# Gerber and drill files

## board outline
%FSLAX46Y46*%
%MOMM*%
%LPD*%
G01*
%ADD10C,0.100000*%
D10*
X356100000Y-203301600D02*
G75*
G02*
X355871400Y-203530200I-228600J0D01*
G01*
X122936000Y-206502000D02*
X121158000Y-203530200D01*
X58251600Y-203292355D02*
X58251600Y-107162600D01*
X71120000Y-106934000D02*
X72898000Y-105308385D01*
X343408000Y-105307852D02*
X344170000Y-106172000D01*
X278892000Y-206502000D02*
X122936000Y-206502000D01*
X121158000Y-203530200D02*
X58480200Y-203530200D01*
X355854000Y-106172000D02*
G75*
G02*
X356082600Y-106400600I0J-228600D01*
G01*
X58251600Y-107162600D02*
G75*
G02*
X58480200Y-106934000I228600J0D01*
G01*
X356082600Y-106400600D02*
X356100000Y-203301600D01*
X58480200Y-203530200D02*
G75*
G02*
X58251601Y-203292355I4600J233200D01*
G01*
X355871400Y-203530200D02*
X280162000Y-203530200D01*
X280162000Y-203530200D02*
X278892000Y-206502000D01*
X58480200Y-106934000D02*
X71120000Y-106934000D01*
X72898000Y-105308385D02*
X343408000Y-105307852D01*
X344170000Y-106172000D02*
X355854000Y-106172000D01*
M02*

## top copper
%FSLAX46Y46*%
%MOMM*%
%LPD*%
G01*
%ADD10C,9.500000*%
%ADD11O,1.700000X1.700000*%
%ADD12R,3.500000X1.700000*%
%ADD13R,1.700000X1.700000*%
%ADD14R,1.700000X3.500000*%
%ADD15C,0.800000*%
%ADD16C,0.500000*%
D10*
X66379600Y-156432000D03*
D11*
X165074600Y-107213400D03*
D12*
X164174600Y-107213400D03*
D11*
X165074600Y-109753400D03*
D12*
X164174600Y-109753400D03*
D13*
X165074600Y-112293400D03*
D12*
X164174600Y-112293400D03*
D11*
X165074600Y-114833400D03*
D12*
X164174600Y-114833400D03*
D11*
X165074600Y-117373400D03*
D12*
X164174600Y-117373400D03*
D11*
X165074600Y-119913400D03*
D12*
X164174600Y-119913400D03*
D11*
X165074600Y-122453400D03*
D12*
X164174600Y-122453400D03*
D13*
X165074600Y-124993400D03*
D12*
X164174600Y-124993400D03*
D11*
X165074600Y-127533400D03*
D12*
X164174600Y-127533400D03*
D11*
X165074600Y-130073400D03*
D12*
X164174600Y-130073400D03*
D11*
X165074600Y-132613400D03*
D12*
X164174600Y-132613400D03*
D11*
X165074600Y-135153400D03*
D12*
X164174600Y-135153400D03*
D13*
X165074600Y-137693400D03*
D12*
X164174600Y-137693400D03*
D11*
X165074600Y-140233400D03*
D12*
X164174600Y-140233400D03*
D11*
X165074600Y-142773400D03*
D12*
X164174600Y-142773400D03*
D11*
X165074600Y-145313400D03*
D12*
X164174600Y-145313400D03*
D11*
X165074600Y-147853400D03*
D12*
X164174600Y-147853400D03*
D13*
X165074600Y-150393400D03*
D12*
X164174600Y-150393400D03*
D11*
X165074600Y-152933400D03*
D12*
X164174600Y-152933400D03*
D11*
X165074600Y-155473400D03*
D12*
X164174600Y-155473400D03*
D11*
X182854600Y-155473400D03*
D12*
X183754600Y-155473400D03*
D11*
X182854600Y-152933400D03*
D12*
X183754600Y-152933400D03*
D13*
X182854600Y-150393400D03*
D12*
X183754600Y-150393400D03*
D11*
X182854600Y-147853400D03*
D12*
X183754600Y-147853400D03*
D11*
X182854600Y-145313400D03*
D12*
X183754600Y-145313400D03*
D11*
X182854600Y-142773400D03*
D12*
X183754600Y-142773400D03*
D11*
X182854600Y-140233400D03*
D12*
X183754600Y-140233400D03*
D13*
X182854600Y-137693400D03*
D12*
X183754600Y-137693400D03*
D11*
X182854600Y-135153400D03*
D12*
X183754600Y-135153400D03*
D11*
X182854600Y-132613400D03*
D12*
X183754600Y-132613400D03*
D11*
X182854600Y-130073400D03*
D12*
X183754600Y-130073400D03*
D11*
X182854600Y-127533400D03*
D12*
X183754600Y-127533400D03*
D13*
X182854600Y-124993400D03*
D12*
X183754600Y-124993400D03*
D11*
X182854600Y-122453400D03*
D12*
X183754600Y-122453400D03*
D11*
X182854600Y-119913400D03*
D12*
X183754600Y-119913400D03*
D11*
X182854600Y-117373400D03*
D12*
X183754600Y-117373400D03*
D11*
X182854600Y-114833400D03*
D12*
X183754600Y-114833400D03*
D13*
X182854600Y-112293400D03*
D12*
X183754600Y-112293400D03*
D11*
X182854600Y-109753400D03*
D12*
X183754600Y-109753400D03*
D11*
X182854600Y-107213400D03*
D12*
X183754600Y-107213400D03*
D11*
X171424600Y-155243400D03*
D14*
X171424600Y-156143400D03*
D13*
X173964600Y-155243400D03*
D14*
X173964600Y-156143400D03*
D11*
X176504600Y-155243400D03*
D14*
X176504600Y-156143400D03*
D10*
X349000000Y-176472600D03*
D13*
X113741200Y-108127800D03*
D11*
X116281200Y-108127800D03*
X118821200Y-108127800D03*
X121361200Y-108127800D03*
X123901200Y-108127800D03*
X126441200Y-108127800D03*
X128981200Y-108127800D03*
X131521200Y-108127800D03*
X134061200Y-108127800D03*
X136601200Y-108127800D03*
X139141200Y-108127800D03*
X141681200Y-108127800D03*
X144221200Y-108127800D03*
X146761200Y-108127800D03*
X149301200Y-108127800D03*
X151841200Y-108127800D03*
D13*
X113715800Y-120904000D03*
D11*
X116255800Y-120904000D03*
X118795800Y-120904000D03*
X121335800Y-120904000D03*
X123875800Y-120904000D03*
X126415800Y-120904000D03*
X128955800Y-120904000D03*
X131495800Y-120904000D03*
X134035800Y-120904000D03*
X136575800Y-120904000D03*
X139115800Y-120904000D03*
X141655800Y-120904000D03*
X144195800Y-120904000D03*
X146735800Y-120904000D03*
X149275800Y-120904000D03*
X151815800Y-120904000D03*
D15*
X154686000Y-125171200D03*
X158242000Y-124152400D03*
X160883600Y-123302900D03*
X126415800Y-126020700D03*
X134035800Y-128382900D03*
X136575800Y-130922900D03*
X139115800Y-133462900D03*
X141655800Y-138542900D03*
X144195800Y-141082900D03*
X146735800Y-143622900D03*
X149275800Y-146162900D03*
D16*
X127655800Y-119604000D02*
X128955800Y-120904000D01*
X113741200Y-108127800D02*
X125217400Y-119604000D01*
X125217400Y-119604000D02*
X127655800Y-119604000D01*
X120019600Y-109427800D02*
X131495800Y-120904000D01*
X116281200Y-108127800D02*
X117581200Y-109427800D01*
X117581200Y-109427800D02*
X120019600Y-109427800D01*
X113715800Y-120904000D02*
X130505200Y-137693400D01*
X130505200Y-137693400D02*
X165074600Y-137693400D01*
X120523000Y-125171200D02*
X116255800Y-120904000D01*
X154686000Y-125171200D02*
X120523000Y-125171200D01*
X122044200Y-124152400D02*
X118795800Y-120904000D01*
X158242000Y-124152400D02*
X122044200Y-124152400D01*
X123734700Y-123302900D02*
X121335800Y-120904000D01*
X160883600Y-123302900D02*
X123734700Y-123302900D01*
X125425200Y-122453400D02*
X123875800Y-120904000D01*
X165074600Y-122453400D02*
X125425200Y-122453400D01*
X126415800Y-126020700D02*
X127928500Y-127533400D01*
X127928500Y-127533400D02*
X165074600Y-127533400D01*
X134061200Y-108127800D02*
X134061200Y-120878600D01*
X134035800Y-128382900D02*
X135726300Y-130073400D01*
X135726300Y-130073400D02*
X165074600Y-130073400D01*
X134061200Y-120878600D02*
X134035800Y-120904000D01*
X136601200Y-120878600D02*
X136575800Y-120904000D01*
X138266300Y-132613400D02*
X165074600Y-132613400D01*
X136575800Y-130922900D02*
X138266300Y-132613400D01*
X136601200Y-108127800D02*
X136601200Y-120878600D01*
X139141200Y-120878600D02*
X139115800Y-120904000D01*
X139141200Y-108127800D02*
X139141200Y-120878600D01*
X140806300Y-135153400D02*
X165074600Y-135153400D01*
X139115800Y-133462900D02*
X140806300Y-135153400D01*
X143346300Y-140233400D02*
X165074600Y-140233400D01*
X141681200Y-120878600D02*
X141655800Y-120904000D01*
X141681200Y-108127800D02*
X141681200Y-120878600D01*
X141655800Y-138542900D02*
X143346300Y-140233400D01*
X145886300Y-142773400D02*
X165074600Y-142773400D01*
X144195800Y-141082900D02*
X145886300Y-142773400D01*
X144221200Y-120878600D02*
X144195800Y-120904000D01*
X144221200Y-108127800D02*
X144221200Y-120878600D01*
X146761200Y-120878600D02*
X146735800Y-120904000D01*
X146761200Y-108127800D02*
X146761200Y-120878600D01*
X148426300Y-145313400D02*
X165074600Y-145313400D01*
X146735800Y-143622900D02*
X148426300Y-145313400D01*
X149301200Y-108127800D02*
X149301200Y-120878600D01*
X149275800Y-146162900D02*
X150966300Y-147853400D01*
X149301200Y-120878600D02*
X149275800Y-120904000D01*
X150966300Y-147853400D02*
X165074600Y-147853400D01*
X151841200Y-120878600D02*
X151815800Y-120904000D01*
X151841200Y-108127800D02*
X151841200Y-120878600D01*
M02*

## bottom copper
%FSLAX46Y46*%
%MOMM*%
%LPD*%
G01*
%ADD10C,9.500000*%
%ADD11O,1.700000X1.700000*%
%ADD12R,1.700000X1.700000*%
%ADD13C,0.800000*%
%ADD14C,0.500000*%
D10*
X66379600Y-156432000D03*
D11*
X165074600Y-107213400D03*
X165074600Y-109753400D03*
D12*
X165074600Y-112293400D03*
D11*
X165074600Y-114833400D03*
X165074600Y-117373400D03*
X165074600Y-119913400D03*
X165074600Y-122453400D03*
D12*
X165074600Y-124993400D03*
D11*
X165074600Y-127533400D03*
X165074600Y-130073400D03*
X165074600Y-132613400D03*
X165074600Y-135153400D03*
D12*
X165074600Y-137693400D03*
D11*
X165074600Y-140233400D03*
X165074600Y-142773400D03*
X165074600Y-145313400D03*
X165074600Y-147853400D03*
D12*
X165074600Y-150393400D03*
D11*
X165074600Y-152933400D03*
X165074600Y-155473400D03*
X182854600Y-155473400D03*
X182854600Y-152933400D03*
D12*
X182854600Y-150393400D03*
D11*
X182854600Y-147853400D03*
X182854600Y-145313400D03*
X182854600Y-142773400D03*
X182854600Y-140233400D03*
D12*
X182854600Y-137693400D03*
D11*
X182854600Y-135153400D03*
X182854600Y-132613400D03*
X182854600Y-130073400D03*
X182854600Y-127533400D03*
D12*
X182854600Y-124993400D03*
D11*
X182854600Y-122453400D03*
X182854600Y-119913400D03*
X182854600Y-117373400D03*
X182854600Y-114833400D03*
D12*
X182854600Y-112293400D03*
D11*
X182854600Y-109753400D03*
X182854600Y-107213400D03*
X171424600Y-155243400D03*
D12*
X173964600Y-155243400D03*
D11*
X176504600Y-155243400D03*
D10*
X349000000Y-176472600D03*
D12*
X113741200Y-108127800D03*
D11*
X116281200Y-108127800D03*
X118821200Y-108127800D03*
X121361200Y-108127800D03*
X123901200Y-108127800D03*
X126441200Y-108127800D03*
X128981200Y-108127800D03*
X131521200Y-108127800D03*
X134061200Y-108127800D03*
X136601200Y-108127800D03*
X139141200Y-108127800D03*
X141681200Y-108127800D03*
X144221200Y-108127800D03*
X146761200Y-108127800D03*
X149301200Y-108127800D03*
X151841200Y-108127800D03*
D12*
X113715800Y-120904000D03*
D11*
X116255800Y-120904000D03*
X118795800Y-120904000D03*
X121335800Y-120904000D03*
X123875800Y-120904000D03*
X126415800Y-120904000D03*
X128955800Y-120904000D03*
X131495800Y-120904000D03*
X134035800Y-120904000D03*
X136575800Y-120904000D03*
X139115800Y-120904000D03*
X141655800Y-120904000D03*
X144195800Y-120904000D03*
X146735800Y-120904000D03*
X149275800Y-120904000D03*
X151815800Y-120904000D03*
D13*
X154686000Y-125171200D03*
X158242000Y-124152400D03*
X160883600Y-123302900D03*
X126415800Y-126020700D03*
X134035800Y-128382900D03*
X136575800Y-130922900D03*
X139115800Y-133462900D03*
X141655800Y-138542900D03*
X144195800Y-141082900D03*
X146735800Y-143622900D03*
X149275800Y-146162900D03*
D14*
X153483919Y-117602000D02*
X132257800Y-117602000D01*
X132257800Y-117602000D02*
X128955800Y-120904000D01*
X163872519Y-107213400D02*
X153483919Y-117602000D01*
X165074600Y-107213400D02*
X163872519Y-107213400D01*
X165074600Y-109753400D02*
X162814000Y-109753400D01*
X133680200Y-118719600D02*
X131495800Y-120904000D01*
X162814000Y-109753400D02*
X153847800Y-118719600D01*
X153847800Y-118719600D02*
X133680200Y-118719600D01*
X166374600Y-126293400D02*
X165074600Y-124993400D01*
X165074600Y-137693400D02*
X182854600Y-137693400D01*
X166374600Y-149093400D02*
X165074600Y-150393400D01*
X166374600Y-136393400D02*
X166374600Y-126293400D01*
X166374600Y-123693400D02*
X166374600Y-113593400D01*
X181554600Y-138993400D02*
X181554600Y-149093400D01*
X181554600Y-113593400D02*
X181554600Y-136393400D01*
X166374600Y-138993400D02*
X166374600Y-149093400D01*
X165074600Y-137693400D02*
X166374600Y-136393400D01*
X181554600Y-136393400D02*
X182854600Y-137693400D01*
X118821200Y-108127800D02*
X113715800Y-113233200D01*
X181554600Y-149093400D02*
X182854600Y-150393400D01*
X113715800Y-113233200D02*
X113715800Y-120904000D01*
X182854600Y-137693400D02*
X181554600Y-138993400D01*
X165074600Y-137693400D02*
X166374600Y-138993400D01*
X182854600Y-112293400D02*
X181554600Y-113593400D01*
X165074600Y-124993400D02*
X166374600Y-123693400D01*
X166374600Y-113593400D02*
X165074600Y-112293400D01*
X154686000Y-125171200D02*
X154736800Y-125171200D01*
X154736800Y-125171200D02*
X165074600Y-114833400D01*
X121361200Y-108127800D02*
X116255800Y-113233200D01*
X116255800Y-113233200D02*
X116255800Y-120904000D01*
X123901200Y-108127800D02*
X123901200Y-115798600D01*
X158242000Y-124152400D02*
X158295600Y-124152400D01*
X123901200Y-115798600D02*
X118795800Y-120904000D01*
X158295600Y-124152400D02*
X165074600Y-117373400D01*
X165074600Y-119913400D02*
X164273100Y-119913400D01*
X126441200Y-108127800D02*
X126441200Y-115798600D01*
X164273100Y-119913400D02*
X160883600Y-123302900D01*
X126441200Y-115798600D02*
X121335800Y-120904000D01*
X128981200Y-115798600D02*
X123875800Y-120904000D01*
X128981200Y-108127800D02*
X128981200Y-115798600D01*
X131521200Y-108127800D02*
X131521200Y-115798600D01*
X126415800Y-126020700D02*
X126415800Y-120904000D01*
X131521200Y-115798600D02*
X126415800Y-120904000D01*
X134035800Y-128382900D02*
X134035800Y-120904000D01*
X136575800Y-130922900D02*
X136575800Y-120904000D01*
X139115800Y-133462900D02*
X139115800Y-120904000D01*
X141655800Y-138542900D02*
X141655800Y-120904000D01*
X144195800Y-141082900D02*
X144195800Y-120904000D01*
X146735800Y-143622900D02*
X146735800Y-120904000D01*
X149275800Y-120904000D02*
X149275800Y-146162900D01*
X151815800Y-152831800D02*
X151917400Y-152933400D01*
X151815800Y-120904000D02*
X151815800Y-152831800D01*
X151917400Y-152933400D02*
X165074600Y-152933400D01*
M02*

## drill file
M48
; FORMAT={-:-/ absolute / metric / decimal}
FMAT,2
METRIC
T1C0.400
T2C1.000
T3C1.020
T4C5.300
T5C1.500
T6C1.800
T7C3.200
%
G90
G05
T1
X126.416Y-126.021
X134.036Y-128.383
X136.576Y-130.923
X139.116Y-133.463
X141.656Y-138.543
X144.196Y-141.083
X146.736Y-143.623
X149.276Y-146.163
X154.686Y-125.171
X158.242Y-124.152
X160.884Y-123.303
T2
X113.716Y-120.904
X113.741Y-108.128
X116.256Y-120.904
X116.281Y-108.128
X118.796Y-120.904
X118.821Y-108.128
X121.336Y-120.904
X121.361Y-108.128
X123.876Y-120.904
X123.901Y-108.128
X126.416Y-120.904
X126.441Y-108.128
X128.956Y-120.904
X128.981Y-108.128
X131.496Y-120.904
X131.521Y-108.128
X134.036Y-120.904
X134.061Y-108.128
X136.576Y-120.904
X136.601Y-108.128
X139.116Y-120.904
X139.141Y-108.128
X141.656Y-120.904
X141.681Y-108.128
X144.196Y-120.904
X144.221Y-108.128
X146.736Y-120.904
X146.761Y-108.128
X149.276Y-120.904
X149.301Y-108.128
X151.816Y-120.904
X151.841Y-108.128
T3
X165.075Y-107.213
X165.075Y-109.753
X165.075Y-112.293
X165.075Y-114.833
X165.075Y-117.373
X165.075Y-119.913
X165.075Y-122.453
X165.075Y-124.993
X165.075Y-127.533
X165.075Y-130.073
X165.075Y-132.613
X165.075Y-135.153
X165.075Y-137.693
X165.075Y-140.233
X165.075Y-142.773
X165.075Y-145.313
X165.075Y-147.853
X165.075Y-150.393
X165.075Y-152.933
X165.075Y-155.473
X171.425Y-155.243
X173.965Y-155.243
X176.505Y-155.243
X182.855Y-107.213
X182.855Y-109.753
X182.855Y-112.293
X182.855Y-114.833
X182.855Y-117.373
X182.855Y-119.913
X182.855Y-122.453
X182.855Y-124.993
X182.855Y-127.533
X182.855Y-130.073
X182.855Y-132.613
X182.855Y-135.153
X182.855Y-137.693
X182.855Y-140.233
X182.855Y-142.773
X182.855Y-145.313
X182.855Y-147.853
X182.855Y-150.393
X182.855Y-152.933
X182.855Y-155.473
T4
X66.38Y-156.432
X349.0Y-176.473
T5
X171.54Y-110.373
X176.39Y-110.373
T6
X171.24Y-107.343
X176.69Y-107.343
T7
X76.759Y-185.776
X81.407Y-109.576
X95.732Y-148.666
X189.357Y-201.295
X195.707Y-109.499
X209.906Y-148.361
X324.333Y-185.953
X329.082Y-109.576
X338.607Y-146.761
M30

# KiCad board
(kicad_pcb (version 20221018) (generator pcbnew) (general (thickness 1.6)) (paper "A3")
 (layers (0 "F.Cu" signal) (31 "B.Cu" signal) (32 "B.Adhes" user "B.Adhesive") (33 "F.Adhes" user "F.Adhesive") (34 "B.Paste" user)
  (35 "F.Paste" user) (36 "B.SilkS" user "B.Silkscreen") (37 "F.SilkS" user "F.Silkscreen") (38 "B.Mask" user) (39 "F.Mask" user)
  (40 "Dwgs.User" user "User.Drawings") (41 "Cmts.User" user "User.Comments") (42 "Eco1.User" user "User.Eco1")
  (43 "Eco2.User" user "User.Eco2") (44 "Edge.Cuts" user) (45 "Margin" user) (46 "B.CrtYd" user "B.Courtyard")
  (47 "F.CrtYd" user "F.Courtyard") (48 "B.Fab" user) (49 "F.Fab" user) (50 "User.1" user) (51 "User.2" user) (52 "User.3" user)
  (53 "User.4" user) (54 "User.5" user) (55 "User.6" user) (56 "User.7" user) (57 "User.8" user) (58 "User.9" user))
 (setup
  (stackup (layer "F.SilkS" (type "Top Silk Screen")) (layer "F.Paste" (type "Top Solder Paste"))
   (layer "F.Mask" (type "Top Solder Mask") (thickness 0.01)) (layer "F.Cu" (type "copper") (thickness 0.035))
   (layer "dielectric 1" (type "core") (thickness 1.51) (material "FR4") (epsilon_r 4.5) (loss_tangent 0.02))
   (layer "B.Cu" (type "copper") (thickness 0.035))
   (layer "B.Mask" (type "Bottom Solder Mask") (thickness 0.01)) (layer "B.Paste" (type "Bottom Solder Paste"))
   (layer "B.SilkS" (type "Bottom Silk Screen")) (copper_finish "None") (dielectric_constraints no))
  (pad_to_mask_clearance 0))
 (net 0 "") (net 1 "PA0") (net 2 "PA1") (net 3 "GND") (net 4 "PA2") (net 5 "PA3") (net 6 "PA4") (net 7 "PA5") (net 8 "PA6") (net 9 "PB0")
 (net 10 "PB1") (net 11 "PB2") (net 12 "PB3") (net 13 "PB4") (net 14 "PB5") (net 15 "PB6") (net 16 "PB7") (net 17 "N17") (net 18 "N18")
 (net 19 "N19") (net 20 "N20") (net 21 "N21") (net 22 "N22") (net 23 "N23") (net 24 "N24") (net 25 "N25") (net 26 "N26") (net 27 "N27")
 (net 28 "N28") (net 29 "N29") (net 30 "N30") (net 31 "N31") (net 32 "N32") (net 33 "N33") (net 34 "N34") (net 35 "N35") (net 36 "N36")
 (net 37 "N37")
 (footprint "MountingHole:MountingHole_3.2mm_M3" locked (layer "F.Cu") (at 189.357 201.295)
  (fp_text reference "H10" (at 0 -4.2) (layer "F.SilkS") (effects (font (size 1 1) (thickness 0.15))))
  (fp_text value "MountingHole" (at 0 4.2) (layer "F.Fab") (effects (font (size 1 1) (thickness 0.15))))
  (pad "" np_thru_hole circle locked (at 0 0) (size 3.2 3.2) (drill 3.2) (layers "*.Cu" "*.Mask")))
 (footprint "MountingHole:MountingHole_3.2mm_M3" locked (layer "F.Cu") (at 209.9056 148.3614)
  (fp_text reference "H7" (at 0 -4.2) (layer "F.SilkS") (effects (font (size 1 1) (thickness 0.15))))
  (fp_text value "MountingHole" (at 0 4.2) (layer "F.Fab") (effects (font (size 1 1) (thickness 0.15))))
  (pad "" np_thru_hole circle locked (at 0 0) (size 3.2 3.2) (drill 3.2) (layers "*.Cu" "*.Mask")))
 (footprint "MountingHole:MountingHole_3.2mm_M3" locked (layer "F.Cu") (at 81.407 109.5756)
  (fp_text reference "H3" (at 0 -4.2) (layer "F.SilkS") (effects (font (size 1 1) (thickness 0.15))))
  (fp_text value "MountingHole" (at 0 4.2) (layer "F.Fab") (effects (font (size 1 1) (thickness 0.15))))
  (pad "" np_thru_hole circle locked (at 0 0) (size 3.2 3.2) (drill 3.2) (layers "*.Cu" "*.Mask")))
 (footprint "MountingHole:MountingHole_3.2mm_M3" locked (layer "F.Cu") (at 329.0824 109.5756)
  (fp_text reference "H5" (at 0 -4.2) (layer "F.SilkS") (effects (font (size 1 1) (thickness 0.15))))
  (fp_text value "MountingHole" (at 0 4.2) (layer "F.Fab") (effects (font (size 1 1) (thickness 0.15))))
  (pad "" np_thru_hole circle locked (at 0 0) (size 3.2 3.2) (drill 3.2) (layers "*.Cu" "*.Mask")))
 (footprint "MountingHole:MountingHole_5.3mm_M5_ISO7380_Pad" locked (layer "F.Cu") (at 66.3796 156.432)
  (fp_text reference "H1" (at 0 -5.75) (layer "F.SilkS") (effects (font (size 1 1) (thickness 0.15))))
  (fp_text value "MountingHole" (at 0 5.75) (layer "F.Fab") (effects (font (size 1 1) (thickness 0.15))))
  (pad "1" thru_hole circle locked (at 0 0) (size 9.5 9.5) (drill 5.3) (layers "*.Cu" "*.Mask")))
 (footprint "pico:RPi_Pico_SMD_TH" (layer "F.Cu") (at 173.9646 131.3434)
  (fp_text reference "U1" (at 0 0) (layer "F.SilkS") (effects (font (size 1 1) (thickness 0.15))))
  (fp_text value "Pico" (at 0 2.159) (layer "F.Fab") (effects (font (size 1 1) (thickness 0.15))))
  (pad "" np_thru_hole oval (at -2.725 -24) (size 1.8 1.8) (drill 1.8) (layers "*.Cu" "*.Mask"))
  (pad "" np_thru_hole oval (at -2.425 -20.97) (size 1.5 1.5) (drill 1.5) (layers "*.Cu" "*.Mask"))
  (pad "" np_thru_hole oval (at 2.425 -20.97) (size 1.5 1.5) (drill 1.5) (layers "*.Cu" "*.Mask"))
  (pad "" np_thru_hole oval (at 2.725 -24) (size 1.8 1.8) (drill 1.8) (layers "*.Cu" "*.Mask"))
  (pad "1" thru_hole oval (at -8.89 -24.13) (size 1.7 1.7) (drill 1.02) (layers "*.Cu" "*.Mask") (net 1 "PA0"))
  (pad "1" smd rect (at -8.89 -24.13) (size 3.5 1.7) (drill (offset -0.9 0)) (layers "F.Cu" "F.Mask") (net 1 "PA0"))
  (pad "2" thru_hole oval (at -8.89 -21.59) (size 1.7 1.7) (drill 1.02) (layers "*.Cu" "*.Mask") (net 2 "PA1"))
  (pad "2" smd rect (at -8.89 -21.59) (size 3.5 1.7) (drill (offset -0.9 0)) (layers "F.Cu" "F.Mask") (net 2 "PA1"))
  (pad "3" thru_hole rect (at -8.89 -19.05) (size 1.7 1.7) (drill 1.02) (layers "*.Cu" "*.Mask") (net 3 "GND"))
  (pad "3" smd rect (at -8.89 -19.05) (size 3.5 1.7) (drill (offset -0.9 0)) (layers "F.Cu" "F.Mask") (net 3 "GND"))
  (pad "4" thru_hole oval (at -8.89 -16.51) (size 1.7 1.7) (drill 1.02) (layers "*.Cu" "*.Mask") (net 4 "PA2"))
  (pad "4" smd rect (at -8.89 -16.51) (size 3.5 1.7) (drill (offset -0.9 0)) (layers "F.Cu" "F.Mask") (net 4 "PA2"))
  (pad "5" thru_hole oval (at -8.89 -13.97) (size 1.7 1.7) (drill 1.02) (layers "*.Cu" "*.Mask") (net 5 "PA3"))
  (pad "5" smd rect (at -8.89 -13.97) (size 3.5 1.7) (drill (offset -0.9 0)) (layers "F.Cu" "F.Mask") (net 5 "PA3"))
  (pad "6" thru_hole oval (at -8.89 -11.43) (size 1.7 1.7) (drill 1.02) (layers "*.Cu" "*.Mask") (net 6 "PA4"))
  (pad "6" smd rect (at -8.89 -11.43) (size 3.5 1.7) (drill (offset -0.9 0)) (layers "F.Cu" "F.Mask") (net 6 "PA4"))
  (pad "7" thru_hole oval (at -8.89 -8.89) (size 1.7 1.7) (drill 1.02) (layers "*.Cu" "*.Mask") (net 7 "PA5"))
  (pad "7" smd rect (at -8.89 -8.89) (size 3.5 1.7) (drill (offset -0.9 0)) (layers "F.Cu" "F.Mask") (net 7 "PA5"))
  (pad "8" thru_hole rect (at -8.89 -6.35) (size 1.7 1.7) (drill 1.02) (layers "*.Cu" "*.Mask") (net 3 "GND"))
  (pad "8" smd rect (at -8.89 -6.35) (size 3.5 1.7) (drill (offset -0.9 0)) (layers "F.Cu" "F.Mask") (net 3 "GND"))
  (pad "9" thru_hole oval (at -8.89 -3.81) (size 1.7 1.7) (drill 1.02) (layers "*.Cu" "*.Mask") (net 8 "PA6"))
  (pad "9" smd rect (at -8.89 -3.81) (size 3.5 1.7) (drill (offset -0.9 0)) (layers "F.Cu" "F.Mask") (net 8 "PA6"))
  (pad "10" thru_hole oval (at -8.89 -1.27) (size 1.7 1.7) (drill 1.02) (layers "*.Cu" "*.Mask") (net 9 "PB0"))
  (pad "10" smd rect (at -8.89 -1.27) (size 3.5 1.7) (drill (offset -0.9 0)) (layers "F.Cu" "F.Mask") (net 9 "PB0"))
  (pad "11" thru_hole oval (at -8.89 1.27) (size 1.7 1.7) (drill 1.02) (layers "*.Cu" "*.Mask") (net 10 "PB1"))
  (pad "11" smd rect (at -8.89 1.27) (size 3.5 1.7) (drill (offset -0.9 0)) (layers "F.Cu" "F.Mask") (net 10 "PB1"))
  (pad "12" thru_hole oval (at -8.89 3.81) (size 1.7 1.7) (drill 1.02) (layers "*.Cu" "*.Mask") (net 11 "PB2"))
  (pad "12" smd rect (at -8.89 3.81) (size 3.5 1.7) (drill (offset -0.9 0)) (layers "F.Cu" "F.Mask") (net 11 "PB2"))
  (pad "13" thru_hole rect (at -8.89 6.35) (size 1.7 1.7) (drill 1.02) (layers "*.Cu" "*.Mask") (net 3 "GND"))
  (pad "13" smd rect (at -8.89 6.35) (size 3.5 1.7) (drill (offset -0.9 0)) (layers "F.Cu" "F.Mask") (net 3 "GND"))
  (pad "14" thru_hole oval (at -8.89 8.89) (size 1.7 1.7) (drill 1.02) (layers "*.Cu" "*.Mask") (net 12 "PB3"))
  (pad "14" smd rect (at -8.89 8.89) (size 3.5 1.7) (drill (offset -0.9 0)) (layers "F.Cu" "F.Mask") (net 12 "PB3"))
  (pad "15" thru_hole oval (at -8.89 11.43) (size 1.7 1.7) (drill 1.02) (layers "*.Cu" "*.Mask") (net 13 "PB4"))
  (pad "15" smd rect (at -8.89 11.43) (size 3.5 1.7) (drill (offset -0.9 0)) (layers "F.Cu" "F.Mask") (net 13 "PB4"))
  (pad "16" thru_hole oval (at -8.89 13.97) (size 1.7 1.7) (drill 1.02) (layers "*.Cu" "*.Mask") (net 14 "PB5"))
  (pad "16" smd rect (at -8.89 13.97) (size 3.5 1.7) (drill (offset -0.9 0)) (layers "F.Cu" "F.Mask") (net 14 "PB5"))
  (pad "17" thru_hole oval (at -8.89 16.51) (size 1.7 1.7) (drill 1.02) (layers "*.Cu" "*.Mask") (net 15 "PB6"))
  (pad "17" smd rect (at -8.89 16.51) (size 3.5 1.7) (drill (offset -0.9 0)) (layers "F.Cu" "F.Mask") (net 15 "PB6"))
  (pad "18" thru_hole rect (at -8.89 19.05) (size 1.7 1.7) (drill 1.02) (layers "*.Cu" "*.Mask") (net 3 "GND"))
  (pad "18" smd rect (at -8.89 19.05) (size 3.5 1.7) (drill (offset -0.9 0)) (layers "F.Cu" "F.Mask") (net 3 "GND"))
  (pad "19" thru_hole oval (at -8.89 21.59) (size 1.7 1.7) (drill 1.02) (layers "*.Cu" "*.Mask") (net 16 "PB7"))
  (pad "19" smd rect (at -8.89 21.59) (size 3.5 1.7) (drill (offset -0.9 0)) (layers "F.Cu" "F.Mask") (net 16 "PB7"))
  (pad "20" thru_hole oval (at -8.89 24.13) (size 1.7 1.7) (drill 1.02) (layers "*.Cu" "*.Mask") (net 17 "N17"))
  (pad "20" smd rect (at -8.89 24.13) (size 3.5 1.7) (drill (offset -0.9 0)) (layers "F.Cu" "F.Mask") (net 17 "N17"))
  (pad "21" thru_hole oval (at 8.89 24.13) (size 1.7 1.7) (drill 1.02) (layers "*.Cu" "*.Mask") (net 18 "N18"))
  (pad "21" smd rect (at 8.89 24.13) (size 3.5 1.7) (drill (offset 0.9 0)) (layers "F.Cu" "F.Mask") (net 18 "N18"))
  (pad "22" thru_hole oval (at 8.89 21.59) (size 1.7 1.7) (drill 1.02) (layers "*.Cu" "*.Mask") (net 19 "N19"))
  (pad "22" smd rect (at 8.89 21.59) (size 3.5 1.7) (drill (offset 0.9 0)) (layers "F.Cu" "F.Mask") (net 19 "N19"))
  (pad "23" thru_hole rect (at 8.89 19.05) (size 1.7 1.7) (drill 1.02) (layers "*.Cu" "*.Mask") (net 3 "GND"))
  (pad "23" smd rect (at 8.89 19.05) (size 3.5 1.7) (drill (offset 0.9 0)) (layers "F.Cu" "F.Mask") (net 3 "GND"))
  (pad "24" thru_hole oval (at 8.89 16.51) (size 1.7 1.7) (drill 1.02) (layers "*.Cu" "*.Mask") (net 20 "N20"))
  (pad "24" smd rect (at 8.89 16.51) (size 3.5 1.7) (drill (offset 0.9 0)) (layers "F.Cu" "F.Mask") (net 20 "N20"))
  (pad "25" thru_hole oval (at 8.89 13.97) (size 1.7 1.7) (drill 1.02) (layers "*.Cu" "*.Mask") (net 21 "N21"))
  (pad "25" smd rect (at 8.89 13.97) (size 3.5 1.7) (drill (offset 0.9 0)) (layers "F.Cu" "F.Mask") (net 21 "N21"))
  (pad "26" thru_hole oval (at 8.89 11.43) (size 1.7 1.7) (drill 1.02) (layers "*.Cu" "*.Mask") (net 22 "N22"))
  (pad "26" smd rect (at 8.89 11.43) (size 3.5 1.7) (drill (offset 0.9 0)) (layers "F.Cu" "F.Mask") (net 22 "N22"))
  (pad "27" thru_hole oval (at 8.89 8.89) (size 1.7 1.7) (drill 1.02) (layers "*.Cu" "*.Mask") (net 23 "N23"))
  (pad "27" smd rect (at 8.89 8.89) (size 3.5 1.7) (drill (offset 0.9 0)) (layers "F.Cu" "F.Mask") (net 23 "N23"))
  (pad "28" thru_hole rect (at 8.89 6.35) (size 1.7 1.7) (drill 1.02) (layers "*.Cu" "*.Mask") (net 3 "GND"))
  (pad "28" smd rect (at 8.89 6.35) (size 3.5 1.7) (drill (offset 0.9 0)) (layers "F.Cu" "F.Mask") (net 3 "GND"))
  (pad "29" thru_hole oval (at 8.89 3.81) (size 1.7 1.7) (drill 1.02) (layers "*.Cu" "*.Mask") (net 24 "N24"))
  (pad "29" smd rect (at 8.89 3.81) (size 3.5 1.7) (drill (offset 0.9 0)) (layers "F.Cu" "F.Mask") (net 24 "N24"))
  (pad "30" thru_hole oval (at 8.89 1.27) (size 1.7 1.7) (drill 1.02) (layers "*.Cu" "*.Mask") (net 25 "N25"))
  (pad "30" smd rect (at 8.89 1.27) (size 3.5 1.7) (drill (offset 0.9 0)) (layers "F.Cu" "F.Mask") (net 25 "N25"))
  (pad "31" thru_hole oval (at 8.89 -1.27) (size 1.7 1.7) (drill 1.02) (layers "*.Cu" "*.Mask") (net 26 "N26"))
  (pad "31" smd rect (at 8.89 -1.27) (size 3.5 1.7) (drill (offset 0.9 0)) (layers "F.Cu" "F.Mask") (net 26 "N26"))
  (pad "32" thru_hole oval (at 8.89 -3.81) (size 1.7 1.7) (drill 1.02) (layers "*.Cu" "*.Mask") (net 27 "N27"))
  (pad "32" smd rect (at 8.89 -3.81) (size 3.5 1.7) (drill (offset 0.9 0)) (layers "F.Cu" "F.Mask") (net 27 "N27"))
  (pad "33" thru_hole rect (at 8.89 -6.35) (size 1.7 1.7) (drill 1.02) (layers "*.Cu" "*.Mask") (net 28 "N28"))
  (pad "33" smd rect (at 8.89 -6.35) (size 3.5 1.7) (drill (offset 0.9 0)) (layers "F.Cu" "F.Mask") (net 28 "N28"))
  (pad "34" thru_hole oval (at 8.89 -8.89) (size 1.7 1.7) (drill 1.02) (layers "*.Cu" "*.Mask") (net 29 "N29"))
  (pad "34" smd rect (at 8.89 -8.89) (size 3.5 1.7) (drill (offset 0.9 0)) (layers "F.Cu" "F.Mask") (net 29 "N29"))
  (pad "35" thru_hole oval (at 8.89 -11.43) (size 1.7 1.7) (drill 1.02) (layers "*.Cu" "*.Mask") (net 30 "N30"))
  (pad "35" smd rect (at 8.89 -11.43) (size 3.5 1.7) (drill (offset 0.9 0)) (layers "F.Cu" "F.Mask") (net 30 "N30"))
  (pad "36" thru_hole oval (at 8.89 -13.97) (size 1.7 1.7) (drill 1.02) (layers "*.Cu" "*.Mask") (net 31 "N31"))
  (pad "36" smd rect (at 8.89 -13.97) (size 3.5 1.7) (drill (offset 0.9 0)) (layers "F.Cu" "F.Mask") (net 31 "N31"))
  (pad "37" thru_hole oval (at 8.89 -16.51) (size 1.7 1.7) (drill 1.02) (layers "*.Cu" "*.Mask") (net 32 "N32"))
  (pad "37" smd rect (at 8.89 -16.51) (size 3.5 1.7) (drill (offset 0.9 0)) (layers "F.Cu" "F.Mask") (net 32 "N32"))
  (pad "38" thru_hole rect (at 8.89 -19.05) (size 1.7 1.7) (drill 1.02) (layers "*.Cu" "*.Mask") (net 3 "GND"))
  (pad "38" smd rect (at 8.89 -19.05) (size 3.5 1.7) (drill (offset 0.9 0)) (layers "F.Cu" "F.Mask") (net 3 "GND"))
  (pad "39" thru_hole oval (at 8.89 -21.59) (size 1.7 1.7) (drill 1.02) (layers "*.Cu" "*.Mask") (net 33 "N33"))
  (pad "39" smd rect (at 8.89 -21.59) (size 3.5 1.7) (drill (offset 0.9 0)) (layers "F.Cu" "F.Mask") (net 33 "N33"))
  (pad "40" thru_hole oval (at 8.89 -24.13) (size 1.7 1.7) (drill 1.02) (layers "*.Cu" "*.Mask") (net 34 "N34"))
  (pad "40" smd rect (at 8.89 -24.13) (size 3.5 1.7) (drill (offset 0.9 0)) (layers "F.Cu" "F.Mask") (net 34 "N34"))
  (pad "41" thru_hole oval (at -2.54 23.9) (size 1.7 1.7) (drill 1.02) (layers "*.Cu" "*.Mask") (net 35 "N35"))
  (pad "41" smd rect (at -2.54 23.9 90) (size 3.5 1.7) (drill (offset -0.9 0)) (layers "F.Cu" "F.Mask") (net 35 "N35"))
  (pad "42" thru_hole rect (at 0 23.9) (size 1.7 1.7) (drill 1.02) (layers "*.Cu" "*.Mask") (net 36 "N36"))
  (pad "42" smd rect (at 0 23.9 90) (size 3.5 1.7) (drill (offset -0.9 0)) (layers "F.Cu" "F.Mask") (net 36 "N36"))
  (pad "43" thru_hole oval (at 2.54 23.9) (size 1.7 1.7) (drill 1.02) (layers "*.Cu" "*.Mask") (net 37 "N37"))
  (pad "43" smd rect (at 2.54 23.9 90) (size 3.5 1.7) (drill (offset -0.9 0)) (layers "F.Cu" "F.Mask") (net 37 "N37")))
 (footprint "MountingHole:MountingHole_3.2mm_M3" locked (layer "F.Cu") (at 338.6074 146.7612)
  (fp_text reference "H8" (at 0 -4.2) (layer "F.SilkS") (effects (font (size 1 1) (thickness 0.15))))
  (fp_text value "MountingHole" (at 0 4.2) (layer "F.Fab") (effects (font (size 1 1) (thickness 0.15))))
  (pad "" np_thru_hole circle locked (at 0 0) (size 3.2 3.2) (drill 3.2) (layers "*.Cu" "*.Mask")))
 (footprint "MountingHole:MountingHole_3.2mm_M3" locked (layer "F.Cu") (at 95.732 148.6662)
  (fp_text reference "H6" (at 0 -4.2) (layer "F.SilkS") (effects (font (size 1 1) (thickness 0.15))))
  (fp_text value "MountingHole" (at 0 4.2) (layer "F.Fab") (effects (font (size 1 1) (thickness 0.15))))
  (pad "" np_thru_hole circle locked (at 0 0) (size 3.2 3.2) (drill 3.2) (layers "*.Cu" "*.Mask")))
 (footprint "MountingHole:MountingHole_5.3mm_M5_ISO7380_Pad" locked (layer "F.Cu") (at 349 176.4726)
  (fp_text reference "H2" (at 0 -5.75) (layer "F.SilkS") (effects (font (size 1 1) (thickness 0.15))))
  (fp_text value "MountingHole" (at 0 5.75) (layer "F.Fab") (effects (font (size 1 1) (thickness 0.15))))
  (pad "1" thru_hole circle locked (at 0 0) (size 9.5 9.5) (drill 5.3) (layers "*.Cu" "*.Mask")))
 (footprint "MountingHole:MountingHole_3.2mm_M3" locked (layer "F.Cu") (at 195.707 109.4994)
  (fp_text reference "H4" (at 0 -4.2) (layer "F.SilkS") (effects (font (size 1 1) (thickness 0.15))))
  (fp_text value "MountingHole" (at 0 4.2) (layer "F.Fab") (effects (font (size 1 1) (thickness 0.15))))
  (pad "" np_thru_hole circle locked (at 0 0) (size 3.2 3.2) (drill 3.2) (layers "*.Cu" "*.Mask")))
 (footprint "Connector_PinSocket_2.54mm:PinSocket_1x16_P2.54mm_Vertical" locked (layer "F.Cu") (at 113.7412 108.1278 90)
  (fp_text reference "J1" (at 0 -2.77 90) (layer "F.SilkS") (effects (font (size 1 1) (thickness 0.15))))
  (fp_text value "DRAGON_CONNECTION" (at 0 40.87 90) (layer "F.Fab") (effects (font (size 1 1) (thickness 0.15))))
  (pad "1" thru_hole rect locked (at 0 0 90) (size 1.7 1.7) (drill 1) (layers "*.Cu" "*.Mask") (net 1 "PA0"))
  (pad "2" thru_hole oval locked (at 0 2.54 90) (size 1.7 1.7) (drill 1) (layers "*.Cu" "*.Mask") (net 2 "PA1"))
  (pad "3" thru_hole oval locked (at 0 5.08 90) (size 1.7 1.7) (drill 1) (layers "*.Cu" "*.Mask") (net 3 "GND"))
  (pad "4" thru_hole oval locked (at 0 7.62 90) (size 1.7 1.7) (drill 1) (layers "*.Cu" "*.Mask") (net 4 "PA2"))
  (pad "5" thru_hole oval locked (at 0 10.16 90) (size 1.7 1.7) (drill 1) (layers "*.Cu" "*.Mask") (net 5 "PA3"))
  (pad "6" thru_hole oval locked (at 0 12.7 90) (size 1.7 1.7) (drill 1) (layers "*.Cu" "*.Mask") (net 6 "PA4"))
  (pad "7" thru_hole oval locked (at 0 15.24 90) (size 1.7 1.7) (drill 1) (layers "*.Cu" "*.Mask") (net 7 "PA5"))
  (pad "8" thru_hole oval locked (at 0 17.78 90) (size 1.7 1.7) (drill 1) (layers "*.Cu" "*.Mask") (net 8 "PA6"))
  (pad "9" thru_hole oval locked (at 0 20.32 90) (size 1.7 1.7) (drill 1) (layers "*.Cu" "*.Mask") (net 9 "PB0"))
  (pad "10" thru_hole oval locked (at 0 22.86 90) (size 1.7 1.7) (drill 1) (layers "*.Cu" "*.Mask") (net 10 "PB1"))
  (pad "11" thru_hole oval locked (at 0 25.4 90) (size 1.7 1.7) (drill 1) (layers "*.Cu" "*.Mask") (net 11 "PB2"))
  (pad "12" thru_hole oval locked (at 0 27.94 90) (size 1.7 1.7) (drill 1) (layers "*.Cu" "*.Mask") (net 12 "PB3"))
  (pad "13" thru_hole oval locked (at 0 30.48 90) (size 1.7 1.7) (drill 1) (layers "*.Cu" "*.Mask") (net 13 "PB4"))
  (pad "14" thru_hole oval locked (at 0 33.02 90) (size 1.7 1.7) (drill 1) (layers "*.Cu" "*.Mask") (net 14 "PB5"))
  (pad "15" thru_hole oval locked (at 0 35.56 90) (size 1.7 1.7) (drill 1) (layers "*.Cu" "*.Mask") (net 15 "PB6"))
  (pad "16" thru_hole oval locked (at 0 38.1 90) (size 1.7 1.7) (drill 1) (layers "*.Cu" "*.Mask") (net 16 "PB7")))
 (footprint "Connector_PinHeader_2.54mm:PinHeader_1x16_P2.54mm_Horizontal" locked (layer "F.Cu") (at 113.7158 120.904 90)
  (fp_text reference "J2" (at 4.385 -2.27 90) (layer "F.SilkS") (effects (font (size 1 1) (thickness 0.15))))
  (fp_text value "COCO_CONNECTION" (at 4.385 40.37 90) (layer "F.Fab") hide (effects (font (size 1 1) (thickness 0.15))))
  (pad "1" thru_hole rect locked (at 0 0 90) (size 1.7 1.7) (drill 1) (layers "*.Cu" "*.Mask") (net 3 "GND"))
  (pad "2" thru_hole oval locked (at 0 2.54 90) (size 1.7 1.7) (drill 1) (layers "*.Cu" "*.Mask") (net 4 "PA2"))
  (pad "3" thru_hole oval locked (at 0 5.08 90) (size 1.7 1.7) (drill 1) (layers "*.Cu" "*.Mask") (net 5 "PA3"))
  (pad "4" thru_hole oval locked (at 0 7.62 90) (size 1.7 1.7) (drill 1) (layers "*.Cu" "*.Mask") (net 6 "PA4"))
  (pad "5" thru_hole oval locked (at 0 10.16 90) (size 1.7 1.7) (drill 1) (layers "*.Cu" "*.Mask") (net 7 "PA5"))
  (pad "6" thru_hole oval locked (at 0 12.7 90) (size 1.7 1.7) (drill 1) (layers "*.Cu" "*.Mask") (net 8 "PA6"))
  (pad "7" thru_hole oval locked (at 0 15.24 90) (size 1.7 1.7) (drill 1) (layers "*.Cu" "*.Mask") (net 1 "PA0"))
  (pad "8" thru_hole oval locked (at 0 17.78 90) (size 1.7 1.7) (drill 1) (layers "*.Cu" "*.Mask") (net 2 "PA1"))
  (pad "9" thru_hole oval locked (at 0 20.32 90) (size 1.7 1.7) (drill 1) (layers "*.Cu" "*.Mask") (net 9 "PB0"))
  (pad "10" thru_hole oval locked (at 0 22.86 90) (size 1.7 1.7) (drill 1) (layers "*.Cu" "*.Mask") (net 10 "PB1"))
  (pad "11" thru_hole oval locked (at 0 25.4 90) (size 1.7 1.7) (drill 1) (layers "*.Cu" "*.Mask") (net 11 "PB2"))
  (pad "12" thru_hole oval locked (at 0 27.94 90) (size 1.7 1.7) (drill 1) (layers "*.Cu" "*.Mask") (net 12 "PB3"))
  (pad "13" thru_hole oval locked (at 0 30.48 90) (size 1.7 1.7) (drill 1) (layers "*.Cu" "*.Mask") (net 13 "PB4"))
  (pad "14" thru_hole oval locked (at 0 33.02 90) (size 1.7 1.7) (drill 1) (layers "*.Cu" "*.Mask") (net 14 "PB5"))
  (pad "15" thru_hole oval locked (at 0 35.56 90) (size 1.7 1.7) (drill 1) (layers "*.Cu" "*.Mask") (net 15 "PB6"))
  (pad "16" thru_hole oval locked (at 0 38.1 90) (size 1.7 1.7) (drill 1) (layers "*.Cu" "*.Mask") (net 16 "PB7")))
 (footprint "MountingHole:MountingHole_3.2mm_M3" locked (layer "F.Cu") (at 324.3326 185.9534)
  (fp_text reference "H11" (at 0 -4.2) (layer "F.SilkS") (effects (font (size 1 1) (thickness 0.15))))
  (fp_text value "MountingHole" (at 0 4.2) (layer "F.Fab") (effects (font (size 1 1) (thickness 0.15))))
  (pad "" np_thru_hole circle locked (at 0 0) (size 3.2 3.2) (drill 3.2) (layers "*.Cu" "*.Mask")))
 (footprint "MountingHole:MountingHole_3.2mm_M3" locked (layer "F.Cu") (at 76.7588 185.7756)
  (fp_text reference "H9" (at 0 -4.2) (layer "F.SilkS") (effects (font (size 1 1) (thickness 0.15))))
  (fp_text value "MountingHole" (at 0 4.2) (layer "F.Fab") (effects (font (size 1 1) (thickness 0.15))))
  (pad "" np_thru_hole circle locked (at 0 0) (size 3.2 3.2) (drill 3.2) (layers "*.Cu" "*.Mask")))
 (gr_arc (start 356.1 203.3016) (mid 356.033045 203.463245) (end 355.8714 203.5302) (stroke (width 0.1) (type default)) (layer "Edge.Cuts"))
 (gr_line (start 122.936 206.502) (end 121.158 203.5302) (stroke (width 0.1) (type default)) (layer "Edge.Cuts"))
 (gr_line (start 58.2516 203.292355) (end 58.2516 107.1626) (stroke (width 0.1) (type default)) (layer "Edge.Cuts"))
 (gr_line (start 71.12 106.934) (end 72.898 105.308385) (stroke (width 0.1) (type default)) (layer "Edge.Cuts"))
 (gr_line (start 343.408 105.307852) (end 344.17 106.172) (stroke (width 0.1) (type default)) (layer "Edge.Cuts"))
 (gr_line (start 278.892 206.502) (end 122.936 206.502) (stroke (width 0.1) (type default)) (layer "Edge.Cuts"))
 (gr_line (start 121.158 203.5302) (end 58.4802 203.5302) (stroke (width 0.1) (type default)) (layer "Edge.Cuts"))
 (gr_arc (start 355.854 106.172) (mid 356.015624 106.238962) (end 356.0826 106.4006) (stroke (width 0.1) (type default)) (layer "Edge.Cuts"))
 (gr_arc (start 58.2516 107.1626) (mid 58.318555 107.000955) (end 58.4802 106.934) (stroke (width 0.1) (type default)) (layer "Edge.Cuts"))
 (gr_line (start 356.0826 106.4006) (end 356.1 203.3016) (stroke (width 0.1) (type default)) (layer "Edge.Cuts"))
 (gr_arc (start 58.4802 203.5302) (mid 58.316634 203.458629) (end 58.2516 203.292355) (stroke (width 0.1) (type default))
  (layer "Edge.Cuts"))
 (gr_line (start 355.8714 203.5302) (end 280.162 203.5302) (stroke (width 0.1) (type default)) (layer "Edge.Cuts"))
 (gr_line (start 280.162 203.5302) (end 278.892 206.502) (stroke (width 0.1) (type default)) (layer "Edge.Cuts"))
 (gr_line (start 58.4802 106.934) (end 71.12 106.934) (stroke (width 0.1) (type default)) (layer "Edge.Cuts"))
 (gr_line (start 72.898 105.308385) (end 343.408 105.307852) (stroke (width 0.1) (type default)) (layer "Edge.Cuts"))
 (gr_line (start 344.17 106.172) (end 355.854 106.172) (stroke (width 0.1) (type default)) (layer "Edge.Cuts"))
 (segment (start 127.6558 119.604) (end 128.9558 120.904) (width 0.5) (layer "F.Cu") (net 1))
 (segment (start 113.7412 108.1278) (end 125.2174 119.604) (width 0.5) (layer "F.Cu") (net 1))
 (segment (start 125.2174 119.604) (end 127.6558 119.604) (width 0.5) (layer "F.Cu") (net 1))
 (segment (start 153.483919 117.602) (end 132.2578 117.602) (width 0.5) (layer "B.Cu") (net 1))
 (segment (start 132.2578 117.602) (end 128.9558 120.904) (width 0.5) (layer "B.Cu") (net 1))
 (segment (start 163.872519 107.2134) (end 153.483919 117.602) (width 0.5) (layer "B.Cu") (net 1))
 (segment (start 165.0746 107.2134) (end 163.872519 107.2134) (width 0.5) (layer "B.Cu") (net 1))
 (segment (start 120.0196 109.4278) (end 131.4958 120.904) (width 0.5) (layer "F.Cu") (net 2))
 (segment (start 116.2812 108.1278) (end 117.5812 109.4278) (width 0.5) (layer "F.Cu") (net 2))
 (segment (start 117.5812 109.4278) (end 120.0196 109.4278) (width 0.5) (layer "F.Cu") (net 2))
 (segment (start 165.0746 109.7534) (end 162.814 109.7534) (width 0.5) (layer "B.Cu") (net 2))
 (segment (start 133.6802 118.7196) (end 131.4958 120.904) (width 0.5) (layer "B.Cu") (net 2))
 (segment (start 162.814 109.7534) (end 153.8478 118.7196) (width 0.5) (layer "B.Cu") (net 2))
 (segment (start 153.8478 118.7196) (end 133.6802 118.7196) (width 0.5) (layer "B.Cu") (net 2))
 (segment (start 113.7158 120.904) (end 130.5052 137.6934) (width 0.5) (layer "F.Cu") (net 3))
 (segment (start 130.5052 137.6934) (end 165.0746 137.6934) (width 0.5) (layer "F.Cu") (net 3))
 (segment (start 166.3746 126.2934) (end 165.0746 124.9934) (width 0.5) (layer "B.Cu") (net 3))
 (segment (start 165.0746 137.6934) (end 182.8546 137.6934) (width 0.5) (layer "B.Cu") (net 3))
 (segment (start 166.3746 149.0934) (end 165.0746 150.3934) (width 0.5) (layer "B.Cu") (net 3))
 (segment (start 166.3746 136.3934) (end 166.3746 126.2934) (width 0.5) (layer "B.Cu") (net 3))
 (segment (start 166.3746 123.6934) (end 166.3746 113.5934) (width 0.5) (layer "B.Cu") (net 3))
 (segment (start 181.5546 138.9934) (end 181.5546 149.0934) (width 0.5) (layer "B.Cu") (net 3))
 (segment (start 181.5546 113.5934) (end 181.5546 136.3934) (width 0.5) (layer "B.Cu") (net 3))
 (segment (start 166.3746 138.9934) (end 166.3746 149.0934) (width 0.5) (layer "B.Cu") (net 3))
 (segment (start 165.0746 137.6934) (end 166.3746 136.3934) (width 0.5) (layer "B.Cu") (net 3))
 (segment (start 181.5546 136.3934) (end 182.8546 137.6934) (width 0.5) (layer "B.Cu") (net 3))
 (segment (start 118.8212 108.1278) (end 113.7158 113.2332) (width 0.5) (layer "B.Cu") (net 3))
 (segment (start 181.5546 149.0934) (end 182.8546 150.3934) (width 0.5) (layer "B.Cu") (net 3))
 (segment (start 113.7158 113.2332) (end 113.7158 120.904) (width 0.5) (layer "B.Cu") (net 3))
 (segment (start 182.8546 137.6934) (end 181.5546 138.9934) (width 0.5) (layer "B.Cu") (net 3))
 (segment (start 165.0746 137.6934) (end 166.3746 138.9934) (width 0.5) (layer "B.Cu") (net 3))
 (segment (start 182.8546 112.2934) (end 181.5546 113.5934) (width 0.5) (layer "B.Cu") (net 3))
 (segment (start 165.0746 124.9934) (end 166.3746 123.6934) (width 0.5) (layer "B.Cu") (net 3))
 (segment (start 166.3746 113.5934) (end 165.0746 112.2934) (width 0.5) (layer "B.Cu") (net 3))
 (segment (start 120.523 125.1712) (end 116.2558 120.904) (width 0.5) (layer "F.Cu") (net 4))
 (segment (start 154.686 125.1712) (end 120.523 125.1712) (width 0.5) (layer "F.Cu") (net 4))
 (via (at 154.686 125.1712) (size 0.8) (drill 0.4) (layers "F.Cu" "B.Cu") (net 4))
 (segment (start 154.686 125.1712) (end 154.7368 125.1712) (width 0.5) (layer "B.Cu") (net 4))
 (segment (start 154.7368 125.1712) (end 165.0746 114.8334) (width 0.5) (layer "B.Cu") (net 4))
 (segment (start 121.3612 108.1278) (end 116.2558 113.2332) (width 0.5) (layer "B.Cu") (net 4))
 (segment (start 116.2558 113.2332) (end 116.2558 120.904) (width 0.5) (layer "B.Cu") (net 4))
 (segment (start 122.0442 124.1524) (end 118.7958 120.904) (width 0.5) (layer "F.Cu") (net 5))
 (segment (start 158.242 124.1524) (end 122.0442 124.1524) (width 0.5) (layer "F.Cu") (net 5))
 (via (at 158.242 124.1524) (size 0.8) (drill 0.4) (layers "F.Cu" "B.Cu") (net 5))
 (segment (start 123.9012 108.1278) (end 123.9012 115.7986) (width 0.5) (layer "B.Cu") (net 5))
 (segment (start 158.242 124.1524) (end 158.2956 124.1524) (width 0.5) (layer "B.Cu") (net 5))
 (segment (start 123.9012 115.7986) (end 118.7958 120.904) (width 0.5) (layer "B.Cu") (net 5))
 (segment (start 158.2956 124.1524) (end 165.0746 117.3734) (width 0.5) (layer "B.Cu") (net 5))
 (segment (start 123.7347 123.3029) (end 121.3358 120.904) (width 0.5) (layer "F.Cu") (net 6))
 (segment (start 160.8836 123.3029) (end 123.7347 123.3029) (width 0.5) (layer "F.Cu") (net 6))
 (via (at 160.8836 123.3029) (size 0.8) (drill 0.4) (layers "F.Cu" "B.Cu") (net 6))
 (segment (start 165.0746 119.9134) (end 164.2731 119.9134) (width 0.5) (layer "B.Cu") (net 6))
 (segment (start 126.4412 108.1278) (end 126.4412 115.7986) (width 0.5) (layer "B.Cu") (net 6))
 (segment (start 164.2731 119.9134) (end 160.8836 123.3029) (width 0.5) (layer "B.Cu") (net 6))
 (segment (start 126.4412 115.7986) (end 121.3358 120.904) (width 0.5) (layer "B.Cu") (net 6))
 (segment (start 125.4252 122.4534) (end 123.8758 120.904) (width 0.5) (layer "F.Cu") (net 7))
 (segment (start 165.0746 122.4534) (end 125.4252 122.4534) (width 0.5) (layer "F.Cu") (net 7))
 (segment (start 128.9812 115.7986) (end 123.8758 120.904) (width 0.5) (layer "B.Cu") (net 7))
 (segment (start 128.9812 108.1278) (end 128.9812 115.7986) (width 0.5) (layer "B.Cu") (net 7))
 (segment (start 126.4158 126.0207) (end 127.9285 127.5334) (width 0.5) (layer "F.Cu") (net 8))
 (segment (start 127.9285 127.5334) (end 165.0746 127.5334) (width 0.5) (layer "F.Cu") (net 8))
 (via (at 126.4158 126.0207) (size 0.8) (drill 0.4) (layers "F.Cu" "B.Cu") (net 8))
 (segment (start 131.5212 108.1278) (end 131.5212 115.7986) (width 0.5) (layer "B.Cu") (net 8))
 (segment (start 126.4158 126.0207) (end 126.4158 120.904) (width 0.5) (layer "B.Cu") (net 8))
 (segment (start 131.5212 115.7986) (end 126.4158 120.904) (width 0.5) (layer "B.Cu") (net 8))
 (segment (start 134.0612 108.1278) (end 134.0612 120.8786) (width 0.5) (layer "F.Cu") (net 9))
 (segment (start 134.0358 128.3829) (end 135.7263 130.0734) (width 0.5) (layer "F.Cu") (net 9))
 (segment (start 135.7263 130.0734) (end 165.0746 130.0734) (width 0.5) (layer "F.Cu") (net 9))
 (segment (start 134.0612 120.8786) (end 134.0358 120.904) (width 0.5) (layer "F.Cu") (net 9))
 (via (at 134.0358 128.3829) (size 0.8) (drill 0.4) (layers "F.Cu" "B.Cu") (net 9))
 (segment (start 134.0358 128.3829) (end 134.0358 120.904) (width 0.5) (layer "B.Cu") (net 9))
 (segment (start 136.6012 120.8786) (end 136.5758 120.904) (width 0.5) (layer "F.Cu") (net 10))
 (segment (start 138.2663 132.6134) (end 165.0746 132.6134) (width 0.5) (layer "F.Cu") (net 10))
 (segment (start 136.5758 130.9229) (end 138.2663 132.6134) (width 0.5) (layer "F.Cu") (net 10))
 (segment (start 136.6012 108.1278) (end 136.6012 120.8786) (width 0.5) (layer "F.Cu") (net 10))
 (via (at 136.5758 130.9229) (size 0.8) (drill 0.4) (layers "F.Cu" "B.Cu") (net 10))
 (segment (start 136.5758 130.9229) (end 136.5758 120.904) (width 0.5) (layer "B.Cu") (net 10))
 (segment (start 139.1412 120.8786) (end 139.1158 120.904) (width 0.5) (layer "F.Cu") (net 11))
 (segment (start 139.1412 108.1278) (end 139.1412 120.8786) (width 0.5) (layer "F.Cu") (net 11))
 (segment (start 140.8063 135.1534) (end 165.0746 135.1534) (width 0.5) (layer "F.Cu") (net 11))
 (segment (start 139.1158 133.4629) (end 140.8063 135.1534) (width 0.5) (layer "F.Cu") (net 11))
 (via (at 139.1158 133.4629) (size 0.8) (drill 0.4) (layers "F.Cu" "B.Cu") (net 11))
 (segment (start 139.1158 133.4629) (end 139.1158 120.904) (width 0.5) (layer "B.Cu") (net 11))
 (segment (start 143.3463 140.2334) (end 165.0746 140.2334) (width 0.5) (layer "F.Cu") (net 12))
 (segment (start 141.6812 120.8786) (end 141.6558 120.904) (width 0.5) (layer "F.Cu") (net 12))
 (segment (start 141.6812 108.1278) (end 141.6812 120.8786) (width 0.5) (layer "F.Cu") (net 12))
 (segment (start 141.6558 138.5429) (end 143.3463 140.2334) (width 0.5) (layer "F.Cu") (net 12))
 (via (at 141.6558 138.5429) (size 0.8) (drill 0.4) (layers "F.Cu" "B.Cu") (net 12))
 (segment (start 141.6558 138.5429) (end 141.6558 120.904) (width 0.5) (layer "B.Cu") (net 12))
 (segment (start 145.8863 142.7734) (end 165.0746 142.7734) (width 0.5) (layer "F.Cu") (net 13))
 (segment (start 144.1958 141.0829) (end 145.8863 142.7734) (width 0.5) (layer "F.Cu") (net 13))
 (segment (start 144.2212 120.8786) (end 144.1958 120.904) (width 0.5) (layer "F.Cu") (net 13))
 (segment (start 144.2212 108.1278) (end 144.2212 120.8786) (width 0.5) (layer "F.Cu") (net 13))
 (via (at 144.1958 141.0829) (size 0.8) (drill 0.4) (layers "F.Cu" "B.Cu") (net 13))
 (segment (start 144.1958 141.0829) (end 144.1958 120.904) (width 0.5) (layer "B.Cu") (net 13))
 (segment (start 146.7612 120.8786) (end 146.7358 120.904) (width 0.5) (layer "F.Cu") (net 14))
 (segment (start 146.7612 108.1278) (end 146.7612 120.8786) (width 0.5) (layer "F.Cu") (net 14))
 (segment (start 148.4263 145.3134) (end 165.0746 145.3134) (width 0.5) (layer "F.Cu") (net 14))
 (segment (start 146.7358 143.6229) (end 148.4263 145.3134) (width 0.5) (layer "F.Cu") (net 14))
 (via (at 146.7358 143.6229) (size 0.8) (drill 0.4) (layers "F.Cu" "B.Cu") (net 14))
 (segment (start 146.7358 143.6229) (end 146.7358 120.904) (width 0.5) (layer "B.Cu") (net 14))
 (segment (start 149.3012 108.1278) (end 149.3012 120.8786) (width 0.5) (layer "F.Cu") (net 15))
 (segment (start 149.2758 146.1629) (end 150.9663 147.8534) (width 0.5) (layer "F.Cu") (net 15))
 (segment (start 149.3012 120.8786) (end 149.2758 120.904) (width 0.5) (layer "F.Cu") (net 15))
 (segment (start 150.9663 147.8534) (end 165.0746 147.8534) (width 0.5) (layer "F.Cu") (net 15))
 (via (at 149.2758 146.1629) (size 0.8) (drill 0.4) (layers "F.Cu" "B.Cu") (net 15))
 (segment (start 149.2758 120.904) (end 149.2758 146.1629) (width 0.5) (layer "B.Cu") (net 15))
 (segment (start 151.8412 120.8786) (end 151.8158 120.904) (width 0.5) (layer "F.Cu") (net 16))
 (segment (start 151.8412 108.1278) (end 151.8412 120.8786) (width 0.5) (layer "F.Cu") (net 16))
 (segment (start 151.8158 152.8318) (end 151.9174 152.9334) (width 0.5) (layer "B.Cu") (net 16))
 (segment (start 151.8158 120.904) (end 151.8158 152.8318) (width 0.5) (layer "B.Cu") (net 16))
 (segment (start 151.9174 152.9334) (end 165.0746 152.9334) (width 0.5) (layer "B.Cu") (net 16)))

